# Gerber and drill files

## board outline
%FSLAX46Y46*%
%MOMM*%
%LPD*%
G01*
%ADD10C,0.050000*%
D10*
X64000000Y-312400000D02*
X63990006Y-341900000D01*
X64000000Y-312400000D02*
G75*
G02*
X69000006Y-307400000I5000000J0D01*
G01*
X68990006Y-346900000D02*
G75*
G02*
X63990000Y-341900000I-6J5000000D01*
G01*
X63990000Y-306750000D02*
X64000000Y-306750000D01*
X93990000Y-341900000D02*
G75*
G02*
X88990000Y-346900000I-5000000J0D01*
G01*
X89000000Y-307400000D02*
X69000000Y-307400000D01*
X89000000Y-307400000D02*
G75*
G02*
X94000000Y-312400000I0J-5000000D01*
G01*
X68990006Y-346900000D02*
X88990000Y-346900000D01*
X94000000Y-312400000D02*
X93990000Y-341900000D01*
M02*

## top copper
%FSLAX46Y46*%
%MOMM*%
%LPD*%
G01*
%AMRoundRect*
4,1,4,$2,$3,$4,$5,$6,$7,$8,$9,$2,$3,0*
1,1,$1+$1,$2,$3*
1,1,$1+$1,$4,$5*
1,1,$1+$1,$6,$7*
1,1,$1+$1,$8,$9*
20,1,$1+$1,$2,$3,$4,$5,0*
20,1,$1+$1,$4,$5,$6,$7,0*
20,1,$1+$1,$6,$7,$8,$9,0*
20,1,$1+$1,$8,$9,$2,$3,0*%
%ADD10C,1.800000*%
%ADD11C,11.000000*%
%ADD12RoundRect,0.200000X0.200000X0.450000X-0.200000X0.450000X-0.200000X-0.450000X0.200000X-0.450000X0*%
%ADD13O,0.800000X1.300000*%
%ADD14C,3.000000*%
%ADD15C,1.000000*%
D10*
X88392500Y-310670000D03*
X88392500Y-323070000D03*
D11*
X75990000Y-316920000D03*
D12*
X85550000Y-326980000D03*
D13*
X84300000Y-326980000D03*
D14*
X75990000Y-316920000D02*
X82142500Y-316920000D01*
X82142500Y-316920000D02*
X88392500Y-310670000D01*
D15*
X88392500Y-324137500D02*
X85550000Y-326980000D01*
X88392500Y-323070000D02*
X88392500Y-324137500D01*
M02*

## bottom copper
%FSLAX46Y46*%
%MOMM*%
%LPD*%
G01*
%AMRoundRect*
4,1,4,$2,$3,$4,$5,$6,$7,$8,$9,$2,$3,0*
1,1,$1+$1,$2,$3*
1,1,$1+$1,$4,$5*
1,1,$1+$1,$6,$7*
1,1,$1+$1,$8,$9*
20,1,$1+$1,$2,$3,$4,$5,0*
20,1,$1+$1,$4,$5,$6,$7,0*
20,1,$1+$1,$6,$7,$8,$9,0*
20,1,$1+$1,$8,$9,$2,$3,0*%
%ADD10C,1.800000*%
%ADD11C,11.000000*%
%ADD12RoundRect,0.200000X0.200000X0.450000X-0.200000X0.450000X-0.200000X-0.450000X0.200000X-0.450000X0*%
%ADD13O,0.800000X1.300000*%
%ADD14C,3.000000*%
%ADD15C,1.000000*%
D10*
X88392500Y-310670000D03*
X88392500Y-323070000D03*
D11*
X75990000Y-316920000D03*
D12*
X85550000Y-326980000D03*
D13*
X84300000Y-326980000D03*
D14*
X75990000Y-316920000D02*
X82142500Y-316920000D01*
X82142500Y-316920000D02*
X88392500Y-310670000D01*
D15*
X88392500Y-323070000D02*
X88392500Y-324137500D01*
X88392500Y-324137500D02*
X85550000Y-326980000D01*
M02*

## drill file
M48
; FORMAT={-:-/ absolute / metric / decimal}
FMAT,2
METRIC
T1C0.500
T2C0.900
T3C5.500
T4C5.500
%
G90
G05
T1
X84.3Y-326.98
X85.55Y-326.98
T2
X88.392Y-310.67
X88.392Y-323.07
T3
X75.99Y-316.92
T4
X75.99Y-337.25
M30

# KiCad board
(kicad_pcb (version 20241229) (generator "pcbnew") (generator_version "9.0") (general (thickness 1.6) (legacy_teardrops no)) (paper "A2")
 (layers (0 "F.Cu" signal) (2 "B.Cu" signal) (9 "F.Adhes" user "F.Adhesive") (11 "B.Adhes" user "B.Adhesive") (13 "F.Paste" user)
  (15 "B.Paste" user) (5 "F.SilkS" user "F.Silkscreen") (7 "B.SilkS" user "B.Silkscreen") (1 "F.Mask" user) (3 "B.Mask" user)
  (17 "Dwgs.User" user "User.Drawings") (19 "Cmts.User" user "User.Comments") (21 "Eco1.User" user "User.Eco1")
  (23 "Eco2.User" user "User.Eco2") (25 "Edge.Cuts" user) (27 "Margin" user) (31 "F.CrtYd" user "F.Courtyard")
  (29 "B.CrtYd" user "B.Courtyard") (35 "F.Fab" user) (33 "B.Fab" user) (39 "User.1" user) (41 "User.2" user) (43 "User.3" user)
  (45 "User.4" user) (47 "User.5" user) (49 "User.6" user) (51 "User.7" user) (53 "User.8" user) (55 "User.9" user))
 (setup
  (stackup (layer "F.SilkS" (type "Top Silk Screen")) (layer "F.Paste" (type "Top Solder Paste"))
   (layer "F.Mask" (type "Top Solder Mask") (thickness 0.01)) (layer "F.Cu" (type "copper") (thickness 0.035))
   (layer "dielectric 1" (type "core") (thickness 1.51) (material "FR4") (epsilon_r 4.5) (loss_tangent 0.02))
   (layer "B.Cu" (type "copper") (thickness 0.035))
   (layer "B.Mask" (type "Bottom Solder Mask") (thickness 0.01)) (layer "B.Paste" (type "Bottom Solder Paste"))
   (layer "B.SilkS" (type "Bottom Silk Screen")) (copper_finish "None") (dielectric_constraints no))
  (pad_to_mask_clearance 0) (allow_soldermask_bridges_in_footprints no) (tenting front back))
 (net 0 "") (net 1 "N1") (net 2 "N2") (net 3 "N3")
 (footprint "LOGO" (layer "F.Cu") (at 90.6 331.53 90)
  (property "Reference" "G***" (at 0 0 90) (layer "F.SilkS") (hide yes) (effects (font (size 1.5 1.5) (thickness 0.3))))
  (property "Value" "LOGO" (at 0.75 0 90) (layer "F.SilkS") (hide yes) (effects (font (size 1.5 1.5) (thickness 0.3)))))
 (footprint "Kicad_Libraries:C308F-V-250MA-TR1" (layer "F.Cu") (at 94.9925 316.27 -90)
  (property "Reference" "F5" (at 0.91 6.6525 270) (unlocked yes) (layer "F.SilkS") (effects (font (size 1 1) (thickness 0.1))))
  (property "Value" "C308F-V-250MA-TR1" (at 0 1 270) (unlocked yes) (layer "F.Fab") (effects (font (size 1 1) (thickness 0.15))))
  (pad "1" thru_hole circle (at -5.6 6.6 270) (size 1.8 1.8) (drill 0.9) (layers "*.Cu" "*.Mask") (remove_unused_layers no) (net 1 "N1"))
  (pad "2" thru_hole circle (at 6.8 6.6 270) (size 1.8 1.8) (drill 0.9) (layers "*.Cu" "*.Mask") (remove_unused_layers no) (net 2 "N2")))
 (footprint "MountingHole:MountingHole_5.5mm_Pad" (layer "F.Cu") (at 75.99 316.92)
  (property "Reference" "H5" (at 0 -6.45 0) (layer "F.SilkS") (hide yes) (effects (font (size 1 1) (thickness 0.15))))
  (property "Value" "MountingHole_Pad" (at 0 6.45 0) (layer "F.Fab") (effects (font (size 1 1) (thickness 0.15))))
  (pad "1" thru_hole circle (at 0 0) (size 11 11) (drill 5.5) (layers "*.Cu" "*.Mask") (remove_unused_layers no) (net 1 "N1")
   (zone_connect 2)))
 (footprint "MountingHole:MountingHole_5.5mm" (layer "F.Cu") (at 75.99 337.25)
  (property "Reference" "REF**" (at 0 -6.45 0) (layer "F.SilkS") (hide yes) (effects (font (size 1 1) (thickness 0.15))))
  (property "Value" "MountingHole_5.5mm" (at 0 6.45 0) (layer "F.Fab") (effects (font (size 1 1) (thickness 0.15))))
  (pad "" np_thru_hole circle (at 0 0) (size 5.5 5.5) (drill 5.5) (layers "*.Cu" "*.Mask")))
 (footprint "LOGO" (layer "F.Cu") (at 90.16 341.13 90)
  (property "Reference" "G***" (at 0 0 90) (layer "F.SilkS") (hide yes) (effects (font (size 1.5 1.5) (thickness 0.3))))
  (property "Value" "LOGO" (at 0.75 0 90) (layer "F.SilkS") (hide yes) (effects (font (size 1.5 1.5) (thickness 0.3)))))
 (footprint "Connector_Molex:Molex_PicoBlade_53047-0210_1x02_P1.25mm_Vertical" (layer "F.Cu") (at 85.55 326.98 180)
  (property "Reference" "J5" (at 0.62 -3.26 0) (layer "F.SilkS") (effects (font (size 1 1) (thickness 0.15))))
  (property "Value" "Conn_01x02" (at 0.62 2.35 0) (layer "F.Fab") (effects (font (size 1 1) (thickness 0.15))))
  (pad "1" thru_hole roundrect (at 0 0 180) (size 0.8 1.3) (drill 0.5) (layers "*.Cu" "*.Mask") (remove_unused_layers no)
   (roundrect_rratio 0.25) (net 2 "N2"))
  (pad "2" thru_hole oval (at 1.25 0 180) (size 0.8 1.3) (drill 0.5) (layers "*.Cu" "*.Mask") (remove_unused_layers no) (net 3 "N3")))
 (gr_line (start 64 312.4) (end 63.990006 341.9) (stroke (width 0.05) (type default)) (layer "Edge.Cuts"))
 (gr_arc (start 64 312.4) (mid 65.464468 308.864464) (end 69.000006 307.4) (stroke (width 0.05) (type default)) (layer "Edge.Cuts"))
 (gr_arc (start 68.990006 346.9) (mid 65.454472 345.435534) (end 63.990006 341.9) (stroke (width 0.05) (type default)) (layer "Edge.Cuts"))
 (gr_line (start 63.99 306.75) (end 64 306.75) (stroke (width 0.05) (type default)) (layer "Edge.Cuts"))
 (gr_arc (start 93.99 341.9) (mid 92.525534 345.435534) (end 88.99 346.9) (stroke (width 0.05) (type default)) (layer "Edge.Cuts"))
 (gr_line (start 89 307.4) (end 69 307.4) (stroke (width 0.05) (type default)) (layer "Edge.Cuts"))
 (gr_arc (start 89 307.4) (mid 92.535534 308.864466) (end 94 312.4) (stroke (width 0.05) (type default)) (layer "Edge.Cuts"))
 (gr_line (start 68.990006 346.9) (end 88.99 346.9) (stroke (width 0.05) (type default)) (layer "Edge.Cuts"))
 (gr_line (start 94 312.4) (end 93.99 341.9) (stroke (width 0.05) (type default)) (layer "Edge.Cuts"))
 (segment (start 75.99 316.92) (end 82.1425 316.92) (width 3) (layer "F.Cu") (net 1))
 (segment (start 82.1425 316.92) (end 88.3925 310.67) (width 3) (layer "F.Cu") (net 1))
 (segment (start 75.99 316.92) (end 82.1425 316.92) (width 3) (layer "B.Cu") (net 1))
 (segment (start 82.1425 316.92) (end 88.3925 310.67) (width 3) (layer "B.Cu") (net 1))
 (segment (start 88.3925 324.1375) (end 85.55 326.98) (width 1) (layer "F.Cu") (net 2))
 (segment (start 88.3925 323.07) (end 88.3925 324.1375) (width 1) (layer "F.Cu") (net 2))
 (segment (start 88.3925 323.07) (end 88.3925 324.1375) (width 1) (layer "B.Cu") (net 2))
 (segment (start 88.3925 324.1375) (end 85.55 326.98) (width 1) (layer "B.Cu") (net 2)))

